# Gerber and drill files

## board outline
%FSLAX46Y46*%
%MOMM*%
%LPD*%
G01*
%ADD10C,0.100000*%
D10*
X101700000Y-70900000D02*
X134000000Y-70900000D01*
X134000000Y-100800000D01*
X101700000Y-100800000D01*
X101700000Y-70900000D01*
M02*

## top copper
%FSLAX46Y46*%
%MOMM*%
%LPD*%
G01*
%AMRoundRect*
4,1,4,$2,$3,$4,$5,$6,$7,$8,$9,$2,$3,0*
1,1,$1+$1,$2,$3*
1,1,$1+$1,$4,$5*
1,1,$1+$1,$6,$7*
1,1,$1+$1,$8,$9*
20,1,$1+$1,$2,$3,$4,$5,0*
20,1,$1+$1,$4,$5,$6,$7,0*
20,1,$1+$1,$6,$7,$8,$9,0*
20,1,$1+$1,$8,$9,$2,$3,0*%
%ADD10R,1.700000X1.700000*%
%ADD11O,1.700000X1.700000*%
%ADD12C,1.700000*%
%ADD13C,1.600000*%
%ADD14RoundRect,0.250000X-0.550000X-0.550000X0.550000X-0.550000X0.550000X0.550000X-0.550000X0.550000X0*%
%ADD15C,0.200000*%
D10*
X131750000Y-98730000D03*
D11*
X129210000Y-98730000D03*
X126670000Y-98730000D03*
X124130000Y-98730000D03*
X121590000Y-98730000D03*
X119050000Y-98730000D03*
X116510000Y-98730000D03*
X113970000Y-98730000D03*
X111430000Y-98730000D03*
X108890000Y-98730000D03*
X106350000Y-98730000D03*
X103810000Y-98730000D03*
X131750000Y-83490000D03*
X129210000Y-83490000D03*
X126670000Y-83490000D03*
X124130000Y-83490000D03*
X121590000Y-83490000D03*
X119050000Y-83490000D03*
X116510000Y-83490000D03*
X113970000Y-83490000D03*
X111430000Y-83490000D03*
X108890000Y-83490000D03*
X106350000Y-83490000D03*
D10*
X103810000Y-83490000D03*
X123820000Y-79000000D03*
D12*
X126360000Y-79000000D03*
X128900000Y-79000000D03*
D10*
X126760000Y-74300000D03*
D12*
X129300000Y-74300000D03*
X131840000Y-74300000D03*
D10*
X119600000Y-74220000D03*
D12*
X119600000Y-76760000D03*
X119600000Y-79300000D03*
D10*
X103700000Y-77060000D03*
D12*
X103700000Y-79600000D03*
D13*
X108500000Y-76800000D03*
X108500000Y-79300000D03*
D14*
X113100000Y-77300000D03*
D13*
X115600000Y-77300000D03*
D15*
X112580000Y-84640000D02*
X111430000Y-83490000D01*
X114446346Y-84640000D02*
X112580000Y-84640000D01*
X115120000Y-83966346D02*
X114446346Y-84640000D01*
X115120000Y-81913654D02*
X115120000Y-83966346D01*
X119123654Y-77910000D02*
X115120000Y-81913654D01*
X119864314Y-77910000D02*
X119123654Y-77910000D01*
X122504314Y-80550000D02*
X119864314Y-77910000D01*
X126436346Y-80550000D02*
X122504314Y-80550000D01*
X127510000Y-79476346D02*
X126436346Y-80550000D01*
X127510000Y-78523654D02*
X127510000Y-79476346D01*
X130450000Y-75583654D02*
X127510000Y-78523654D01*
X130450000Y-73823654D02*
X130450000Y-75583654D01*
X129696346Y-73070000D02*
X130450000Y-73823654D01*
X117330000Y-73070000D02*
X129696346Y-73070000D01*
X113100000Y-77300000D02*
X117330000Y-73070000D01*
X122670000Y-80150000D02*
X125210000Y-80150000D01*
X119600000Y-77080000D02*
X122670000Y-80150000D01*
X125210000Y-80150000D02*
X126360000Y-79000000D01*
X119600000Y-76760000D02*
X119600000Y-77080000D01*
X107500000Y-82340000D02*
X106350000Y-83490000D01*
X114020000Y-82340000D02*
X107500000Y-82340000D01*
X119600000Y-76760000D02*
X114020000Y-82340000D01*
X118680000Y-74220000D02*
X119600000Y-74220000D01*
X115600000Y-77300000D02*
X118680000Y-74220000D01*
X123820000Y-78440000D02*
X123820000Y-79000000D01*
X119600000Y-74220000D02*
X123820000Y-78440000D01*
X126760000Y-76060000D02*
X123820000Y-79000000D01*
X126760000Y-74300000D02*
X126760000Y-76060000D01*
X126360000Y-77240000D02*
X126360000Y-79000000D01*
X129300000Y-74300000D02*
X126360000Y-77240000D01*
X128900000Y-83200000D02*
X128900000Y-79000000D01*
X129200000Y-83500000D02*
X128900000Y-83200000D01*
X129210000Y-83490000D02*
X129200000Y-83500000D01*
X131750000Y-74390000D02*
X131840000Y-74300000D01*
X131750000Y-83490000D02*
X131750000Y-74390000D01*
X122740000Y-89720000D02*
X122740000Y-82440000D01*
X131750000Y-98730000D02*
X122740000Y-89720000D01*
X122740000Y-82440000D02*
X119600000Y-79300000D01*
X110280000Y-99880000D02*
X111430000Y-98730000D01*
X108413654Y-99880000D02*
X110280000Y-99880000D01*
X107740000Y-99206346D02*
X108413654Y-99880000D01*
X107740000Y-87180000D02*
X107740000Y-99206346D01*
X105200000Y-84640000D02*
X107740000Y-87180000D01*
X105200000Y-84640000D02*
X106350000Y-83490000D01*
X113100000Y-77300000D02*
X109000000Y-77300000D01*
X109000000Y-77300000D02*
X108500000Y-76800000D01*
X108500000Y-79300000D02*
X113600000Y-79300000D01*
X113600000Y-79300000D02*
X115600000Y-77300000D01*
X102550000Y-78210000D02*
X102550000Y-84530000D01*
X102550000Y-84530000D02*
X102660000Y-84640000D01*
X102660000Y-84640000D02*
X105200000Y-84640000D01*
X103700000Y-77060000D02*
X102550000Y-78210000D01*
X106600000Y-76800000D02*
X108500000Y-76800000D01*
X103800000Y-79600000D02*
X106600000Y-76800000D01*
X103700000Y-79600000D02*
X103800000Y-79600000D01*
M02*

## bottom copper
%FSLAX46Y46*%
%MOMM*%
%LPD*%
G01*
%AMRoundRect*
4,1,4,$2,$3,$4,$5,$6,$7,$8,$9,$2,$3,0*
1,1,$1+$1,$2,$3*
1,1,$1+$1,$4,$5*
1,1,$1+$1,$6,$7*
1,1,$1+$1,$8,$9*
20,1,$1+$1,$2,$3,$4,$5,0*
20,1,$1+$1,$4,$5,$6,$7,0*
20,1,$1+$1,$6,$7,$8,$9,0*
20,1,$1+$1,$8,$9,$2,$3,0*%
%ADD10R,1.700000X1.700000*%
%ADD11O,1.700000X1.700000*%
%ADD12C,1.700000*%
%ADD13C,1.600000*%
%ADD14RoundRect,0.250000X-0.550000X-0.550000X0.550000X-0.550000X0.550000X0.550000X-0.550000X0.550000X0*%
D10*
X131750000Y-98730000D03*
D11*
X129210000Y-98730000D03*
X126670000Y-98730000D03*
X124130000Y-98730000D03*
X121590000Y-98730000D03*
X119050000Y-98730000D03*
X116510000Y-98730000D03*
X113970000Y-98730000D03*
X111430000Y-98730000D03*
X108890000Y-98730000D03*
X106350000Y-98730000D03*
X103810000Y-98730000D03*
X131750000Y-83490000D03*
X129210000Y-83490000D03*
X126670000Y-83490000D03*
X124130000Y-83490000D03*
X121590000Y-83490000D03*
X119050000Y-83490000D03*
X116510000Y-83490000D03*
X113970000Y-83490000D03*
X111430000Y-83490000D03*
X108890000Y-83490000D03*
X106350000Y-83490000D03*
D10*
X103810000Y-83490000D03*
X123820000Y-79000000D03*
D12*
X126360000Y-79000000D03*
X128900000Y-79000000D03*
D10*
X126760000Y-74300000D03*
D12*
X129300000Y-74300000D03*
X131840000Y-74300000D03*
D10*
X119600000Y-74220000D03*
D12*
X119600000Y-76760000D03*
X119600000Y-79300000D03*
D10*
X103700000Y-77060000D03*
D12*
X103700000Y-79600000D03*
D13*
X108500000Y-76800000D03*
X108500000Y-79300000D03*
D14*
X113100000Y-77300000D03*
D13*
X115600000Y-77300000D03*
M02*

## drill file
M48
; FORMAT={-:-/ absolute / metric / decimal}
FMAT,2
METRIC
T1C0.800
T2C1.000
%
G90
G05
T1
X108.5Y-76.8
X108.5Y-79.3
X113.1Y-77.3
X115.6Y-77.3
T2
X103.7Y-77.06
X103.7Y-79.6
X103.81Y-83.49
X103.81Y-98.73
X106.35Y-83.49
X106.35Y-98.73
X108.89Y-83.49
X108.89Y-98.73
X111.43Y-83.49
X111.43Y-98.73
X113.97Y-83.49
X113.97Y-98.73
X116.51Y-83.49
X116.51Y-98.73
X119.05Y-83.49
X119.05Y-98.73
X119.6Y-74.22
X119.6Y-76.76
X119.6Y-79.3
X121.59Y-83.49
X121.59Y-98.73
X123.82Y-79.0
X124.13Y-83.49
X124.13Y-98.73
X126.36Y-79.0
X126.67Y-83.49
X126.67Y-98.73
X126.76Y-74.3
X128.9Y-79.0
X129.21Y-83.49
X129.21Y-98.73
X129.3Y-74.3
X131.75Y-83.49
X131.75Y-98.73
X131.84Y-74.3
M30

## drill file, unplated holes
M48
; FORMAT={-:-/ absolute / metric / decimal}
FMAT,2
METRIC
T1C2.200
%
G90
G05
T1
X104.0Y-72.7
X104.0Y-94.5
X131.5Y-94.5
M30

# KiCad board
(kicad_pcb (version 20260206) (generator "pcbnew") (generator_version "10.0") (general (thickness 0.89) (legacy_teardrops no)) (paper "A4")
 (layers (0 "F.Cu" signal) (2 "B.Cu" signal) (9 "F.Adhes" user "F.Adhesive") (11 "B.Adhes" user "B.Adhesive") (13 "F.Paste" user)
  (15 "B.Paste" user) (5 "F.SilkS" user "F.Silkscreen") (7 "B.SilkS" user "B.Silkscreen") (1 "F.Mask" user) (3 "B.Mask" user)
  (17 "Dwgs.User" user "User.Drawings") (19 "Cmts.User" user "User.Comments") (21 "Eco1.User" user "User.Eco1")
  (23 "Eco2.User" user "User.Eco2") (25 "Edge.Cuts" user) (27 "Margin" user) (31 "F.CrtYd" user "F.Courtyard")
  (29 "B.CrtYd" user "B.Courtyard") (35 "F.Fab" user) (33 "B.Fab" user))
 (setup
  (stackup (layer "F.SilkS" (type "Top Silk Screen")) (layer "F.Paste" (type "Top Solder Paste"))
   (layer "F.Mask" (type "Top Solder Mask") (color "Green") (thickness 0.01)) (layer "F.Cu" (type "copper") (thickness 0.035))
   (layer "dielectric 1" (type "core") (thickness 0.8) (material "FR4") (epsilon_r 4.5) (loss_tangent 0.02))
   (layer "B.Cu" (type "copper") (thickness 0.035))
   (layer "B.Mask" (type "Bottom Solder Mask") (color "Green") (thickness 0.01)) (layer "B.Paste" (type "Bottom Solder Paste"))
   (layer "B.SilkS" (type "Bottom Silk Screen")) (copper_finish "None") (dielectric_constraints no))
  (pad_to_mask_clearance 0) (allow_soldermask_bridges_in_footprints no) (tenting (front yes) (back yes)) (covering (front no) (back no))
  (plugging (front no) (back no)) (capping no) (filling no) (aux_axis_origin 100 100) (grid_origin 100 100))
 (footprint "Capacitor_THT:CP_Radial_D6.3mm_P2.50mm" (layer "F.Cu") (at 113.1 77.3)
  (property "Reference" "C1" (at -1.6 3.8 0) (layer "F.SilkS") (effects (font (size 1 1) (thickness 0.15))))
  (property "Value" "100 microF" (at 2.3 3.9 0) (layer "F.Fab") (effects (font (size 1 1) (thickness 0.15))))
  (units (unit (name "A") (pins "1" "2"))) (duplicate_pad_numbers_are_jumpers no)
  (pad "1" thru_hole roundrect (at 0 0) (size 1.6 1.6) (drill 0.8) (layers "*.Cu" "*.Mask") (remove_unused_layers no)
   (roundrect_rratio 0.15625) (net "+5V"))
  (pad "2" thru_hole circle (at 2.5 0) (size 1.6 1.6) (drill 0.8) (layers "*.Cu" "*.Mask") (remove_unused_layers no) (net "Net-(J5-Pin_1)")))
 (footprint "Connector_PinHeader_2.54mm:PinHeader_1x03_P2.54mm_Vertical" (layer "F.Cu") (at 119.6 74.22)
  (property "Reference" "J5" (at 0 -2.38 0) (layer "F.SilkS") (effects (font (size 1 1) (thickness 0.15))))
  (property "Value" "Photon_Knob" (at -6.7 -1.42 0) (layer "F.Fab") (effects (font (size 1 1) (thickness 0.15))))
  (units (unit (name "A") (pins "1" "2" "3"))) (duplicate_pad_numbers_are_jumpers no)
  (pad "1" thru_hole rect (at 0 0) (size 1.7 1.7) (drill 1) (layers "*.Cu" "*.Mask") (remove_unused_layers no) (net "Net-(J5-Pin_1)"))
  (pad "2" thru_hole circle (at 0 2.54) (size 1.7 1.7) (drill 1) (layers "*.Cu" "*.Mask") (remove_unused_layers no) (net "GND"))
  (pad "3" thru_hole circle (at 0 5.08) (size 1.7 1.7) (drill 1) (layers "*.Cu" "*.Mask") (remove_unused_layers no) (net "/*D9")))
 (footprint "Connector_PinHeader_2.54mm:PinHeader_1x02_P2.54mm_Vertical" (layer "F.Cu") (at 103.7 77.06)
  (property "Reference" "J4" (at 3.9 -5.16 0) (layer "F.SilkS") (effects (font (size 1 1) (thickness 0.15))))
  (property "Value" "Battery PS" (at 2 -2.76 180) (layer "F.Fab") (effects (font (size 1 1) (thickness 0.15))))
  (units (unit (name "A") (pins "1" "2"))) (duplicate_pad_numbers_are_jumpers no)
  (pad "1" thru_hole rect (at 0 0) (size 1.7 1.7) (drill 1) (layers "*.Cu" "*.Mask") (remove_unused_layers no) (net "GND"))
  (pad "2" thru_hole circle (at 0 2.54) (size 1.7 1.7) (drill 1) (layers "*.Cu" "*.Mask") (remove_unused_layers no) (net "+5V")))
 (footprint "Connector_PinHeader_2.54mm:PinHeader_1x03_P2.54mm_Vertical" (layer "F.Cu") (at 126.76 74.3 90)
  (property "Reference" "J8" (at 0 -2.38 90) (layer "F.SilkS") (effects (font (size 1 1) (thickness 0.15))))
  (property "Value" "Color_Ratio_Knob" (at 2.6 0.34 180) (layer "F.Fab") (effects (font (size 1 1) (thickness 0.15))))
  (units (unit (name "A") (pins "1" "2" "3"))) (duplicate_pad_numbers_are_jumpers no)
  (pad "1" thru_hole rect (at 0 0 90) (size 1.7 1.7) (drill 1) (layers "*.Cu" "*.Mask") (remove_unused_layers no) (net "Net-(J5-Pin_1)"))
  (pad "2" thru_hole circle (at 0 2.54 90) (size 1.7 1.7) (drill 1) (layers "*.Cu" "*.Mask") (remove_unused_layers no) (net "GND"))
  (pad "3" thru_hole circle (at 0 5.08 90) (size 1.7 1.7) (drill 1) (layers "*.Cu" "*.Mask") (remove_unused_layers no)
   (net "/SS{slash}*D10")))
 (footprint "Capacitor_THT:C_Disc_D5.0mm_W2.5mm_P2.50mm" (layer "F.Cu") (at 108.5 76.8 -90)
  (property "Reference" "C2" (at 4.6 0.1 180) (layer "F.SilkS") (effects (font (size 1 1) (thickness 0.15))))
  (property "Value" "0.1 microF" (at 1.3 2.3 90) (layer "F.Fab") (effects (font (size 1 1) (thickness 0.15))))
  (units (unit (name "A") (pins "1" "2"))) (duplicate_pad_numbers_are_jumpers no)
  (pad "1" thru_hole circle (at 0 0 270) (size 1.6 1.6) (drill 0.8) (layers "*.Cu" "*.Mask") (remove_unused_layers no) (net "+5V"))
  (pad "2" thru_hole circle (at 2.5 0 270) (size 1.6 1.6) (drill 0.8) (layers "*.Cu" "*.Mask") (remove_unused_layers no)
   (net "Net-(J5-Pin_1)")))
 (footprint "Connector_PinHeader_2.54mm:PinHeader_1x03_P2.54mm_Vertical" (layer "F.Cu") (at 123.82 79 90)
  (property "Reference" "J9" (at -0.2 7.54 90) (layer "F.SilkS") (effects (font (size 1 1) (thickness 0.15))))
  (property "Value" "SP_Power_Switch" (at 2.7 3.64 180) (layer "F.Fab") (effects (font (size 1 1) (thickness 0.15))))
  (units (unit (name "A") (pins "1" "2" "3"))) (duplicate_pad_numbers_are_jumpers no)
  (pad "1" thru_hole rect (at 0 0 90) (size 1.7 1.7) (drill 1) (layers "*.Cu" "*.Mask") (remove_unused_layers no) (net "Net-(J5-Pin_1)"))
  (pad "2" thru_hole circle (at 0 2.54 90) (size 1.7 1.7) (drill 1) (layers "*.Cu" "*.Mask") (remove_unused_layers no) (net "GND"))
  (pad "3" thru_hole circle (at 0 5.08 90) (size 1.7 1.7) (drill 1) (layers "*.Cu" "*.Mask") (remove_unused_layers no)
   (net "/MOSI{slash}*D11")))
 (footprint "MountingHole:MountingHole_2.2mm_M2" (layer "F.Cu") (at 131.5 94.5)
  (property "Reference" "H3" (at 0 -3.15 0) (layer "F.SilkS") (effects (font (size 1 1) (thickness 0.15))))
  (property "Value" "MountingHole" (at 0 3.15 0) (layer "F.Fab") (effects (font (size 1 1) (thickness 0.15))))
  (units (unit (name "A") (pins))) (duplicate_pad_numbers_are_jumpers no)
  (pad "" np_thru_hole circle (at 0 0) (size 2.2 2.2) (drill 2.2) (layers "*.Cu" "*.Mask")))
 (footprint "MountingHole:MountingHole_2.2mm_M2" (layer "F.Cu") (at 104 72.7)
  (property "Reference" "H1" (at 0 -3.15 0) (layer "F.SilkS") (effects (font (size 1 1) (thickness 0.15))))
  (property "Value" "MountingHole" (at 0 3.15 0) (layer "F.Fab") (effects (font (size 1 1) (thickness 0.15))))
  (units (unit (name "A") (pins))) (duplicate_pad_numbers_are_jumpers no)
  (pad "" np_thru_hole circle (at 0 0) (size 2.2 2.2) (drill 2.2) (layers "*.Cu" "*.Mask")))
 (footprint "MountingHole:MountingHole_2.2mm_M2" (layer "F.Cu") (at 104 94.5)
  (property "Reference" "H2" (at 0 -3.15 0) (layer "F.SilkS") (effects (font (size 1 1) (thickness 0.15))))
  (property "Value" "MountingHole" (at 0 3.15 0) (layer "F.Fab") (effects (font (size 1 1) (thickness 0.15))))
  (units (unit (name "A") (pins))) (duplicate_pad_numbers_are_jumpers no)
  (pad "" np_thru_hole circle (at 0 0) (size 2.2 2.2) (drill 2.2) (layers "*.Cu" "*.Mask")))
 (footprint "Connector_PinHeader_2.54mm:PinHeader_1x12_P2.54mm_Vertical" (layer "B.Cu") (at 131.75 98.73 90)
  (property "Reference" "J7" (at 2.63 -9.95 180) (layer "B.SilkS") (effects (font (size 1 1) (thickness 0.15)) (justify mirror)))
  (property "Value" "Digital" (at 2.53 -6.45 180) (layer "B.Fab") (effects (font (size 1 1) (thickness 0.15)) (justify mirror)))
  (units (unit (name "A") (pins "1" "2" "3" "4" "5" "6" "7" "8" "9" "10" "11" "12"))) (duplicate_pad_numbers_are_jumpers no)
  (pad "1" thru_hole rect (at 0 0 90) (size 1.7 1.7) (drill 1) (layers "*.Cu" "*.Mask") (remove_unused_layers no) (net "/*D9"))
  (pad "2" thru_hole oval (at 0 -2.54 90) (size 1.7 1.7) (drill 1) (layers "*.Cu" "*.Mask") (remove_unused_layers no) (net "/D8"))
  (pad "3" thru_hole oval (at 0 -5.08 90) (size 1.7 1.7) (drill 1) (layers "*.Cu" "*.Mask") (remove_unused_layers no) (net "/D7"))
  (pad "4" thru_hole oval (at 0 -7.62 90) (size 1.7 1.7) (drill 1) (layers "*.Cu" "*.Mask") (remove_unused_layers no) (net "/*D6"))
  (pad "5" thru_hole oval (at 0 -10.16 90) (size 1.7 1.7) (drill 1) (layers "*.Cu" "*.Mask") (remove_unused_layers no) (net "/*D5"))
  (pad "6" thru_hole oval (at 0 -12.7 90) (size 1.7 1.7) (drill 1) (layers "*.Cu" "*.Mask") (remove_unused_layers no) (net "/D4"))
  (pad "7" thru_hole oval (at 0 -15.24 90) (size 1.7 1.7) (drill 1) (layers "*.Cu" "*.Mask") (remove_unused_layers no) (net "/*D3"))
  (pad "8" thru_hole oval (at 0 -17.78 90) (size 1.7 1.7) (drill 1) (layers "*.Cu" "*.Mask") (remove_unused_layers no) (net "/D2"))
  (pad "9" thru_hole oval (at 0 -20.32 90) (size 1.7 1.7) (drill 1) (layers "*.Cu" "*.Mask") (remove_unused_layers no) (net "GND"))
  (pad "10" thru_hole oval (at 0 -22.86 90) (size 1.7 1.7) (drill 1) (layers "*.Cu" "*.Mask") (remove_unused_layers no)
   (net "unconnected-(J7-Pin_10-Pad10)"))
  (pad "11" thru_hole oval (at 0 -25.4 90) (size 1.7 1.7) (drill 1) (layers "*.Cu" "*.Mask") (remove_unused_layers no) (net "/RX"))
  (pad "12" thru_hole oval (at 0 -27.94 90) (size 1.7 1.7) (drill 1) (layers "*.Cu" "*.Mask") (remove_unused_layers no) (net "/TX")))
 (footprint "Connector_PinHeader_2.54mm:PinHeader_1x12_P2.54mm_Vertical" (layer "B.Cu") (at 103.81 83.49 -90)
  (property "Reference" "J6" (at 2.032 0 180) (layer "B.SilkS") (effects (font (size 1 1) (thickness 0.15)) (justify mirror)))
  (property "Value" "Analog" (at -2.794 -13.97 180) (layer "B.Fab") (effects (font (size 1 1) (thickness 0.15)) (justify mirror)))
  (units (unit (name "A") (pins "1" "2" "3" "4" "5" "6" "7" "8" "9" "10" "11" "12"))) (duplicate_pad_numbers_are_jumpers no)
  (pad "1" thru_hole rect (at 0 0 270) (size 1.7 1.7) (drill 1) (layers "*.Cu" "*.Mask") (remove_unused_layers no) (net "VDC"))
  (pad "2" thru_hole oval (at 0 -2.54 270) (size 1.7 1.7) (drill 1) (layers "*.Cu" "*.Mask") (remove_unused_layers no) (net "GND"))
  (pad "3" thru_hole oval (at 0 -5.08 270) (size 1.7 1.7) (drill 1) (layers "*.Cu" "*.Mask") (remove_unused_layers no)
   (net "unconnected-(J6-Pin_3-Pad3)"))
  (pad "4" thru_hole oval (at 0 -7.62 270) (size 1.7 1.7) (drill 1) (layers "*.Cu" "*.Mask") (remove_unused_layers no) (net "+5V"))
  (pad "5" thru_hole oval (at 0 -10.16 270) (size 1.7 1.7) (drill 1) (layers "*.Cu" "*.Mask") (remove_unused_layers no) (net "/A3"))
  (pad "6" thru_hole oval (at 0 -12.7 270) (size 1.7 1.7) (drill 1) (layers "*.Cu" "*.Mask") (remove_unused_layers no) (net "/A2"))
  (pad "7" thru_hole oval (at 0 -15.24 270) (size 1.7 1.7) (drill 1) (layers "*.Cu" "*.Mask") (remove_unused_layers no) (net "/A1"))
  (pad "8" thru_hole oval (at 0 -17.78 270) (size 1.7 1.7) (drill 1) (layers "*.Cu" "*.Mask") (remove_unused_layers no) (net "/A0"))
  (pad "9" thru_hole oval (at 0 -20.32 270) (size 1.7 1.7) (drill 1) (layers "*.Cu" "*.Mask") (remove_unused_layers no)
   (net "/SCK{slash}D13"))
  (pad "10" thru_hole oval (at 0 -22.86 270) (size 1.7 1.7) (drill 1) (layers "*.Cu" "*.Mask") (remove_unused_layers no)
   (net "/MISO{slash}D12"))
  (pad "11" thru_hole oval (at 0 -25.4 270) (size 1.7 1.7) (drill 1) (layers "*.Cu" "*.Mask") (remove_unused_layers no)
   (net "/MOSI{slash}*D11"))
  (pad "12" thru_hole oval (at 0 -27.94 270) (size 1.7 1.7) (drill 1) (layers "*.Cu" "*.Mask") (remove_unused_layers no)
   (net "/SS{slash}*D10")))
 (gr_rect (start 101.7 70.9) (end 134 100.8) (stroke (width 0.1) (type default)) (fill no) (layer "Edge.Cuts"))
 (segment (start 115.12 81.913654) (end 115.12 83.966346) (width 0.2) (layer "F.Cu") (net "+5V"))
 (segment (start 115.12 83.966346) (end 114.446346 84.64) (width 0.2) (layer "F.Cu") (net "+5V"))
 (segment (start 103.8 79.6) (end 106.6 76.8) (width 0.2) (layer "F.Cu") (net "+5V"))
 (segment (start 114.446346 84.64) (end 112.58 84.64) (width 0.2) (layer "F.Cu") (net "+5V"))
 (segment (start 130.45 75.583654) (end 127.51 78.523654) (width 0.2) (layer "F.Cu") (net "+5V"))
 (segment (start 122.504314 80.55) (end 119.864314 77.91) (width 0.2) (layer "F.Cu") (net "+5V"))
 (segment (start 126.436346 80.55) (end 122.504314 80.55) (width 0.2) (layer "F.Cu") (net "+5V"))
 (segment (start 129.696346 73.07) (end 130.45 73.823654) (width 0.2) (layer "F.Cu") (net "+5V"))
 (segment (start 113.1 77.3) (end 117.33 73.07) (width 0.2) (layer "F.Cu") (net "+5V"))
 (segment (start 127.51 78.523654) (end 127.51 79.476346) (width 0.2) (layer "F.Cu") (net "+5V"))
 (segment (start 113.1 77.3) (end 109 77.3) (width 0.2) (layer "F.Cu") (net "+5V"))
 (segment (start 119.123654 77.91) (end 115.12 81.913654) (width 0.2) (layer "F.Cu") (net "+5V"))
 (segment (start 119.864314 77.91) (end 119.123654 77.91) (width 0.2) (layer "F.Cu") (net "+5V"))
 (segment (start 130.45 73.823654) (end 130.45 75.583654) (width 0.2) (layer "F.Cu") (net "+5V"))
 (segment (start 117.33 73.07) (end 129.696346 73.07) (width 0.2) (layer "F.Cu") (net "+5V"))
 (segment (start 112.58 84.64) (end 111.43 83.49) (width 0.2) (layer "F.Cu") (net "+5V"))
 (segment (start 109 77.3) (end 108.5 76.8) (width 0.2) (layer "F.Cu") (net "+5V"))
 (segment (start 103.7 79.6) (end 103.8 79.6) (width 0.2) (layer "F.Cu") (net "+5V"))
 (segment (start 127.51 79.476346) (end 126.436346 80.55) (width 0.2) (layer "F.Cu") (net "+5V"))
 (segment (start 106.6 76.8) (end 108.5 76.8) (width 0.2) (layer "F.Cu") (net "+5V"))
 (segment (start 123.82 78.44) (end 123.82 79) (width 0.2) (layer "F.Cu") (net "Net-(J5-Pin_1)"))
 (segment (start 113.6 79.3) (end 115.6 77.3) (width 0.2) (layer "F.Cu") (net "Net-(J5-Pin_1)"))
 (segment (start 115.6 77.3) (end 118.68 74.22) (width 0.2) (layer "F.Cu") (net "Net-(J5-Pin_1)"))
 (segment (start 119.6 74.22) (end 123.82 78.44) (width 0.2) (layer "F.Cu") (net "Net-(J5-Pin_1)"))
 (segment (start 126.76 76.06) (end 123.82 79) (width 0.2) (layer "F.Cu") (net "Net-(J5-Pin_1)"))
 (segment (start 108.5 79.3) (end 113.6 79.3) (width 0.2) (layer "F.Cu") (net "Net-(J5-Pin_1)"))
 (segment (start 118.68 74.22) (end 119.6 74.22) (width 0.2) (layer "F.Cu") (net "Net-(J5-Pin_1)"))
 (segment (start 126.76 74.3) (end 126.76 76.06) (width 0.2) (layer "F.Cu") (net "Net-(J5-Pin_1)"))
 (segment (start 110.28 99.88) (end 111.43 98.73) (width 0.2) (layer "F.Cu") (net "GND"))
 (segment (start 107.74 87.18) (end 107.74 99.206346) (width 0.2) (layer "F.Cu") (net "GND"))
 (segment (start 105.2 84.64) (end 106.35 83.49) (width 0.2) (layer "F.Cu") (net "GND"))
 (segment (start 102.55 84.53) (end 102.66 84.64) (width 0.2) (layer "F.Cu") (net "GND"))
 (segment (start 107.5 82.34) (end 106.35 83.49) (width 0.2) (layer "F.Cu") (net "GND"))
 (segment (start 114.02 82.34) (end 107.5 82.34) (width 0.2) (layer "F.Cu") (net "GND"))
 (segment (start 108.413654 99.88) (end 110.28 99.88) (width 0.2) (layer "F.Cu") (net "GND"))
 (segment (start 119.6 76.76) (end 114.02 82.34) (width 0.2) (layer "F.Cu") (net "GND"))
 (segment (start 122.67 80.15) (end 125.21 80.15) (width 0.2) (layer "F.Cu") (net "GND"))
 (segment (start 102.55 78.21) (end 102.55 84.53) (width 0.2) (layer "F.Cu") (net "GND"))
 (segment (start 126.36 77.24) (end 126.36 79) (width 0.2) (layer "F.Cu") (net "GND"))
 (segment (start 107.74 99.206346) (end 108.413654 99.88) (width 0.2) (layer "F.Cu") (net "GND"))
 (segment (start 125.21 80.15) (end 126.36 79) (width 0.2) (layer "F.Cu") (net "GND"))
 (segment (start 102.66 84.64) (end 105.2 84.64) (width 0.2) (layer "F.Cu") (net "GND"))
 (segment (start 105.2 84.64) (end 107.74 87.18) (width 0.2) (layer "F.Cu") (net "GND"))
 (segment (start 129.3 74.3) (end 126.36 77.24) (width 0.2) (layer "F.Cu") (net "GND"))
 (segment (start 119.6 76.76) (end 119.6 77.08) (width 0.2) (layer "F.Cu") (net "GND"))
 (segment (start 103.7 77.06) (end 102.55 78.21) (width 0.2) (layer "F.Cu") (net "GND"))
 (segment (start 119.6 77.08) (end 122.67 80.15) (width 0.2) (layer "F.Cu") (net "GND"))
 (segment (start 122.74 89.72) (end 122.74 82.44) (width 0.2) (layer "F.Cu") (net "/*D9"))
 (segment (start 131.75 98.73) (end 122.74 89.72) (width 0.2) (layer "F.Cu") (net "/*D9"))
 (segment (start 122.74 82.44) (end 119.6 79.3) (width 0.2) (layer "F.Cu") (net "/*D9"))
 (segment (start 131.75 83.49) (end 131.75 74.39) (width 0.2) (layer "F.Cu") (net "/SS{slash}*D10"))
 (segment (start 131.75 74.39) (end 131.84 74.3) (width 0.2) (layer "F.Cu") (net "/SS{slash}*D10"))
 (segment (start 128.9 83.2) (end 128.9 79) (width 0.2) (layer "F.Cu") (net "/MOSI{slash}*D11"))
 (segment (start 129.21 83.49) (end 129.2 83.5) (width 0.2) (layer "F.Cu") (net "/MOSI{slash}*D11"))
 (segment (start 129.2 83.5) (end 128.9 83.2) (width 0.2) (layer "F.Cu") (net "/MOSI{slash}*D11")))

